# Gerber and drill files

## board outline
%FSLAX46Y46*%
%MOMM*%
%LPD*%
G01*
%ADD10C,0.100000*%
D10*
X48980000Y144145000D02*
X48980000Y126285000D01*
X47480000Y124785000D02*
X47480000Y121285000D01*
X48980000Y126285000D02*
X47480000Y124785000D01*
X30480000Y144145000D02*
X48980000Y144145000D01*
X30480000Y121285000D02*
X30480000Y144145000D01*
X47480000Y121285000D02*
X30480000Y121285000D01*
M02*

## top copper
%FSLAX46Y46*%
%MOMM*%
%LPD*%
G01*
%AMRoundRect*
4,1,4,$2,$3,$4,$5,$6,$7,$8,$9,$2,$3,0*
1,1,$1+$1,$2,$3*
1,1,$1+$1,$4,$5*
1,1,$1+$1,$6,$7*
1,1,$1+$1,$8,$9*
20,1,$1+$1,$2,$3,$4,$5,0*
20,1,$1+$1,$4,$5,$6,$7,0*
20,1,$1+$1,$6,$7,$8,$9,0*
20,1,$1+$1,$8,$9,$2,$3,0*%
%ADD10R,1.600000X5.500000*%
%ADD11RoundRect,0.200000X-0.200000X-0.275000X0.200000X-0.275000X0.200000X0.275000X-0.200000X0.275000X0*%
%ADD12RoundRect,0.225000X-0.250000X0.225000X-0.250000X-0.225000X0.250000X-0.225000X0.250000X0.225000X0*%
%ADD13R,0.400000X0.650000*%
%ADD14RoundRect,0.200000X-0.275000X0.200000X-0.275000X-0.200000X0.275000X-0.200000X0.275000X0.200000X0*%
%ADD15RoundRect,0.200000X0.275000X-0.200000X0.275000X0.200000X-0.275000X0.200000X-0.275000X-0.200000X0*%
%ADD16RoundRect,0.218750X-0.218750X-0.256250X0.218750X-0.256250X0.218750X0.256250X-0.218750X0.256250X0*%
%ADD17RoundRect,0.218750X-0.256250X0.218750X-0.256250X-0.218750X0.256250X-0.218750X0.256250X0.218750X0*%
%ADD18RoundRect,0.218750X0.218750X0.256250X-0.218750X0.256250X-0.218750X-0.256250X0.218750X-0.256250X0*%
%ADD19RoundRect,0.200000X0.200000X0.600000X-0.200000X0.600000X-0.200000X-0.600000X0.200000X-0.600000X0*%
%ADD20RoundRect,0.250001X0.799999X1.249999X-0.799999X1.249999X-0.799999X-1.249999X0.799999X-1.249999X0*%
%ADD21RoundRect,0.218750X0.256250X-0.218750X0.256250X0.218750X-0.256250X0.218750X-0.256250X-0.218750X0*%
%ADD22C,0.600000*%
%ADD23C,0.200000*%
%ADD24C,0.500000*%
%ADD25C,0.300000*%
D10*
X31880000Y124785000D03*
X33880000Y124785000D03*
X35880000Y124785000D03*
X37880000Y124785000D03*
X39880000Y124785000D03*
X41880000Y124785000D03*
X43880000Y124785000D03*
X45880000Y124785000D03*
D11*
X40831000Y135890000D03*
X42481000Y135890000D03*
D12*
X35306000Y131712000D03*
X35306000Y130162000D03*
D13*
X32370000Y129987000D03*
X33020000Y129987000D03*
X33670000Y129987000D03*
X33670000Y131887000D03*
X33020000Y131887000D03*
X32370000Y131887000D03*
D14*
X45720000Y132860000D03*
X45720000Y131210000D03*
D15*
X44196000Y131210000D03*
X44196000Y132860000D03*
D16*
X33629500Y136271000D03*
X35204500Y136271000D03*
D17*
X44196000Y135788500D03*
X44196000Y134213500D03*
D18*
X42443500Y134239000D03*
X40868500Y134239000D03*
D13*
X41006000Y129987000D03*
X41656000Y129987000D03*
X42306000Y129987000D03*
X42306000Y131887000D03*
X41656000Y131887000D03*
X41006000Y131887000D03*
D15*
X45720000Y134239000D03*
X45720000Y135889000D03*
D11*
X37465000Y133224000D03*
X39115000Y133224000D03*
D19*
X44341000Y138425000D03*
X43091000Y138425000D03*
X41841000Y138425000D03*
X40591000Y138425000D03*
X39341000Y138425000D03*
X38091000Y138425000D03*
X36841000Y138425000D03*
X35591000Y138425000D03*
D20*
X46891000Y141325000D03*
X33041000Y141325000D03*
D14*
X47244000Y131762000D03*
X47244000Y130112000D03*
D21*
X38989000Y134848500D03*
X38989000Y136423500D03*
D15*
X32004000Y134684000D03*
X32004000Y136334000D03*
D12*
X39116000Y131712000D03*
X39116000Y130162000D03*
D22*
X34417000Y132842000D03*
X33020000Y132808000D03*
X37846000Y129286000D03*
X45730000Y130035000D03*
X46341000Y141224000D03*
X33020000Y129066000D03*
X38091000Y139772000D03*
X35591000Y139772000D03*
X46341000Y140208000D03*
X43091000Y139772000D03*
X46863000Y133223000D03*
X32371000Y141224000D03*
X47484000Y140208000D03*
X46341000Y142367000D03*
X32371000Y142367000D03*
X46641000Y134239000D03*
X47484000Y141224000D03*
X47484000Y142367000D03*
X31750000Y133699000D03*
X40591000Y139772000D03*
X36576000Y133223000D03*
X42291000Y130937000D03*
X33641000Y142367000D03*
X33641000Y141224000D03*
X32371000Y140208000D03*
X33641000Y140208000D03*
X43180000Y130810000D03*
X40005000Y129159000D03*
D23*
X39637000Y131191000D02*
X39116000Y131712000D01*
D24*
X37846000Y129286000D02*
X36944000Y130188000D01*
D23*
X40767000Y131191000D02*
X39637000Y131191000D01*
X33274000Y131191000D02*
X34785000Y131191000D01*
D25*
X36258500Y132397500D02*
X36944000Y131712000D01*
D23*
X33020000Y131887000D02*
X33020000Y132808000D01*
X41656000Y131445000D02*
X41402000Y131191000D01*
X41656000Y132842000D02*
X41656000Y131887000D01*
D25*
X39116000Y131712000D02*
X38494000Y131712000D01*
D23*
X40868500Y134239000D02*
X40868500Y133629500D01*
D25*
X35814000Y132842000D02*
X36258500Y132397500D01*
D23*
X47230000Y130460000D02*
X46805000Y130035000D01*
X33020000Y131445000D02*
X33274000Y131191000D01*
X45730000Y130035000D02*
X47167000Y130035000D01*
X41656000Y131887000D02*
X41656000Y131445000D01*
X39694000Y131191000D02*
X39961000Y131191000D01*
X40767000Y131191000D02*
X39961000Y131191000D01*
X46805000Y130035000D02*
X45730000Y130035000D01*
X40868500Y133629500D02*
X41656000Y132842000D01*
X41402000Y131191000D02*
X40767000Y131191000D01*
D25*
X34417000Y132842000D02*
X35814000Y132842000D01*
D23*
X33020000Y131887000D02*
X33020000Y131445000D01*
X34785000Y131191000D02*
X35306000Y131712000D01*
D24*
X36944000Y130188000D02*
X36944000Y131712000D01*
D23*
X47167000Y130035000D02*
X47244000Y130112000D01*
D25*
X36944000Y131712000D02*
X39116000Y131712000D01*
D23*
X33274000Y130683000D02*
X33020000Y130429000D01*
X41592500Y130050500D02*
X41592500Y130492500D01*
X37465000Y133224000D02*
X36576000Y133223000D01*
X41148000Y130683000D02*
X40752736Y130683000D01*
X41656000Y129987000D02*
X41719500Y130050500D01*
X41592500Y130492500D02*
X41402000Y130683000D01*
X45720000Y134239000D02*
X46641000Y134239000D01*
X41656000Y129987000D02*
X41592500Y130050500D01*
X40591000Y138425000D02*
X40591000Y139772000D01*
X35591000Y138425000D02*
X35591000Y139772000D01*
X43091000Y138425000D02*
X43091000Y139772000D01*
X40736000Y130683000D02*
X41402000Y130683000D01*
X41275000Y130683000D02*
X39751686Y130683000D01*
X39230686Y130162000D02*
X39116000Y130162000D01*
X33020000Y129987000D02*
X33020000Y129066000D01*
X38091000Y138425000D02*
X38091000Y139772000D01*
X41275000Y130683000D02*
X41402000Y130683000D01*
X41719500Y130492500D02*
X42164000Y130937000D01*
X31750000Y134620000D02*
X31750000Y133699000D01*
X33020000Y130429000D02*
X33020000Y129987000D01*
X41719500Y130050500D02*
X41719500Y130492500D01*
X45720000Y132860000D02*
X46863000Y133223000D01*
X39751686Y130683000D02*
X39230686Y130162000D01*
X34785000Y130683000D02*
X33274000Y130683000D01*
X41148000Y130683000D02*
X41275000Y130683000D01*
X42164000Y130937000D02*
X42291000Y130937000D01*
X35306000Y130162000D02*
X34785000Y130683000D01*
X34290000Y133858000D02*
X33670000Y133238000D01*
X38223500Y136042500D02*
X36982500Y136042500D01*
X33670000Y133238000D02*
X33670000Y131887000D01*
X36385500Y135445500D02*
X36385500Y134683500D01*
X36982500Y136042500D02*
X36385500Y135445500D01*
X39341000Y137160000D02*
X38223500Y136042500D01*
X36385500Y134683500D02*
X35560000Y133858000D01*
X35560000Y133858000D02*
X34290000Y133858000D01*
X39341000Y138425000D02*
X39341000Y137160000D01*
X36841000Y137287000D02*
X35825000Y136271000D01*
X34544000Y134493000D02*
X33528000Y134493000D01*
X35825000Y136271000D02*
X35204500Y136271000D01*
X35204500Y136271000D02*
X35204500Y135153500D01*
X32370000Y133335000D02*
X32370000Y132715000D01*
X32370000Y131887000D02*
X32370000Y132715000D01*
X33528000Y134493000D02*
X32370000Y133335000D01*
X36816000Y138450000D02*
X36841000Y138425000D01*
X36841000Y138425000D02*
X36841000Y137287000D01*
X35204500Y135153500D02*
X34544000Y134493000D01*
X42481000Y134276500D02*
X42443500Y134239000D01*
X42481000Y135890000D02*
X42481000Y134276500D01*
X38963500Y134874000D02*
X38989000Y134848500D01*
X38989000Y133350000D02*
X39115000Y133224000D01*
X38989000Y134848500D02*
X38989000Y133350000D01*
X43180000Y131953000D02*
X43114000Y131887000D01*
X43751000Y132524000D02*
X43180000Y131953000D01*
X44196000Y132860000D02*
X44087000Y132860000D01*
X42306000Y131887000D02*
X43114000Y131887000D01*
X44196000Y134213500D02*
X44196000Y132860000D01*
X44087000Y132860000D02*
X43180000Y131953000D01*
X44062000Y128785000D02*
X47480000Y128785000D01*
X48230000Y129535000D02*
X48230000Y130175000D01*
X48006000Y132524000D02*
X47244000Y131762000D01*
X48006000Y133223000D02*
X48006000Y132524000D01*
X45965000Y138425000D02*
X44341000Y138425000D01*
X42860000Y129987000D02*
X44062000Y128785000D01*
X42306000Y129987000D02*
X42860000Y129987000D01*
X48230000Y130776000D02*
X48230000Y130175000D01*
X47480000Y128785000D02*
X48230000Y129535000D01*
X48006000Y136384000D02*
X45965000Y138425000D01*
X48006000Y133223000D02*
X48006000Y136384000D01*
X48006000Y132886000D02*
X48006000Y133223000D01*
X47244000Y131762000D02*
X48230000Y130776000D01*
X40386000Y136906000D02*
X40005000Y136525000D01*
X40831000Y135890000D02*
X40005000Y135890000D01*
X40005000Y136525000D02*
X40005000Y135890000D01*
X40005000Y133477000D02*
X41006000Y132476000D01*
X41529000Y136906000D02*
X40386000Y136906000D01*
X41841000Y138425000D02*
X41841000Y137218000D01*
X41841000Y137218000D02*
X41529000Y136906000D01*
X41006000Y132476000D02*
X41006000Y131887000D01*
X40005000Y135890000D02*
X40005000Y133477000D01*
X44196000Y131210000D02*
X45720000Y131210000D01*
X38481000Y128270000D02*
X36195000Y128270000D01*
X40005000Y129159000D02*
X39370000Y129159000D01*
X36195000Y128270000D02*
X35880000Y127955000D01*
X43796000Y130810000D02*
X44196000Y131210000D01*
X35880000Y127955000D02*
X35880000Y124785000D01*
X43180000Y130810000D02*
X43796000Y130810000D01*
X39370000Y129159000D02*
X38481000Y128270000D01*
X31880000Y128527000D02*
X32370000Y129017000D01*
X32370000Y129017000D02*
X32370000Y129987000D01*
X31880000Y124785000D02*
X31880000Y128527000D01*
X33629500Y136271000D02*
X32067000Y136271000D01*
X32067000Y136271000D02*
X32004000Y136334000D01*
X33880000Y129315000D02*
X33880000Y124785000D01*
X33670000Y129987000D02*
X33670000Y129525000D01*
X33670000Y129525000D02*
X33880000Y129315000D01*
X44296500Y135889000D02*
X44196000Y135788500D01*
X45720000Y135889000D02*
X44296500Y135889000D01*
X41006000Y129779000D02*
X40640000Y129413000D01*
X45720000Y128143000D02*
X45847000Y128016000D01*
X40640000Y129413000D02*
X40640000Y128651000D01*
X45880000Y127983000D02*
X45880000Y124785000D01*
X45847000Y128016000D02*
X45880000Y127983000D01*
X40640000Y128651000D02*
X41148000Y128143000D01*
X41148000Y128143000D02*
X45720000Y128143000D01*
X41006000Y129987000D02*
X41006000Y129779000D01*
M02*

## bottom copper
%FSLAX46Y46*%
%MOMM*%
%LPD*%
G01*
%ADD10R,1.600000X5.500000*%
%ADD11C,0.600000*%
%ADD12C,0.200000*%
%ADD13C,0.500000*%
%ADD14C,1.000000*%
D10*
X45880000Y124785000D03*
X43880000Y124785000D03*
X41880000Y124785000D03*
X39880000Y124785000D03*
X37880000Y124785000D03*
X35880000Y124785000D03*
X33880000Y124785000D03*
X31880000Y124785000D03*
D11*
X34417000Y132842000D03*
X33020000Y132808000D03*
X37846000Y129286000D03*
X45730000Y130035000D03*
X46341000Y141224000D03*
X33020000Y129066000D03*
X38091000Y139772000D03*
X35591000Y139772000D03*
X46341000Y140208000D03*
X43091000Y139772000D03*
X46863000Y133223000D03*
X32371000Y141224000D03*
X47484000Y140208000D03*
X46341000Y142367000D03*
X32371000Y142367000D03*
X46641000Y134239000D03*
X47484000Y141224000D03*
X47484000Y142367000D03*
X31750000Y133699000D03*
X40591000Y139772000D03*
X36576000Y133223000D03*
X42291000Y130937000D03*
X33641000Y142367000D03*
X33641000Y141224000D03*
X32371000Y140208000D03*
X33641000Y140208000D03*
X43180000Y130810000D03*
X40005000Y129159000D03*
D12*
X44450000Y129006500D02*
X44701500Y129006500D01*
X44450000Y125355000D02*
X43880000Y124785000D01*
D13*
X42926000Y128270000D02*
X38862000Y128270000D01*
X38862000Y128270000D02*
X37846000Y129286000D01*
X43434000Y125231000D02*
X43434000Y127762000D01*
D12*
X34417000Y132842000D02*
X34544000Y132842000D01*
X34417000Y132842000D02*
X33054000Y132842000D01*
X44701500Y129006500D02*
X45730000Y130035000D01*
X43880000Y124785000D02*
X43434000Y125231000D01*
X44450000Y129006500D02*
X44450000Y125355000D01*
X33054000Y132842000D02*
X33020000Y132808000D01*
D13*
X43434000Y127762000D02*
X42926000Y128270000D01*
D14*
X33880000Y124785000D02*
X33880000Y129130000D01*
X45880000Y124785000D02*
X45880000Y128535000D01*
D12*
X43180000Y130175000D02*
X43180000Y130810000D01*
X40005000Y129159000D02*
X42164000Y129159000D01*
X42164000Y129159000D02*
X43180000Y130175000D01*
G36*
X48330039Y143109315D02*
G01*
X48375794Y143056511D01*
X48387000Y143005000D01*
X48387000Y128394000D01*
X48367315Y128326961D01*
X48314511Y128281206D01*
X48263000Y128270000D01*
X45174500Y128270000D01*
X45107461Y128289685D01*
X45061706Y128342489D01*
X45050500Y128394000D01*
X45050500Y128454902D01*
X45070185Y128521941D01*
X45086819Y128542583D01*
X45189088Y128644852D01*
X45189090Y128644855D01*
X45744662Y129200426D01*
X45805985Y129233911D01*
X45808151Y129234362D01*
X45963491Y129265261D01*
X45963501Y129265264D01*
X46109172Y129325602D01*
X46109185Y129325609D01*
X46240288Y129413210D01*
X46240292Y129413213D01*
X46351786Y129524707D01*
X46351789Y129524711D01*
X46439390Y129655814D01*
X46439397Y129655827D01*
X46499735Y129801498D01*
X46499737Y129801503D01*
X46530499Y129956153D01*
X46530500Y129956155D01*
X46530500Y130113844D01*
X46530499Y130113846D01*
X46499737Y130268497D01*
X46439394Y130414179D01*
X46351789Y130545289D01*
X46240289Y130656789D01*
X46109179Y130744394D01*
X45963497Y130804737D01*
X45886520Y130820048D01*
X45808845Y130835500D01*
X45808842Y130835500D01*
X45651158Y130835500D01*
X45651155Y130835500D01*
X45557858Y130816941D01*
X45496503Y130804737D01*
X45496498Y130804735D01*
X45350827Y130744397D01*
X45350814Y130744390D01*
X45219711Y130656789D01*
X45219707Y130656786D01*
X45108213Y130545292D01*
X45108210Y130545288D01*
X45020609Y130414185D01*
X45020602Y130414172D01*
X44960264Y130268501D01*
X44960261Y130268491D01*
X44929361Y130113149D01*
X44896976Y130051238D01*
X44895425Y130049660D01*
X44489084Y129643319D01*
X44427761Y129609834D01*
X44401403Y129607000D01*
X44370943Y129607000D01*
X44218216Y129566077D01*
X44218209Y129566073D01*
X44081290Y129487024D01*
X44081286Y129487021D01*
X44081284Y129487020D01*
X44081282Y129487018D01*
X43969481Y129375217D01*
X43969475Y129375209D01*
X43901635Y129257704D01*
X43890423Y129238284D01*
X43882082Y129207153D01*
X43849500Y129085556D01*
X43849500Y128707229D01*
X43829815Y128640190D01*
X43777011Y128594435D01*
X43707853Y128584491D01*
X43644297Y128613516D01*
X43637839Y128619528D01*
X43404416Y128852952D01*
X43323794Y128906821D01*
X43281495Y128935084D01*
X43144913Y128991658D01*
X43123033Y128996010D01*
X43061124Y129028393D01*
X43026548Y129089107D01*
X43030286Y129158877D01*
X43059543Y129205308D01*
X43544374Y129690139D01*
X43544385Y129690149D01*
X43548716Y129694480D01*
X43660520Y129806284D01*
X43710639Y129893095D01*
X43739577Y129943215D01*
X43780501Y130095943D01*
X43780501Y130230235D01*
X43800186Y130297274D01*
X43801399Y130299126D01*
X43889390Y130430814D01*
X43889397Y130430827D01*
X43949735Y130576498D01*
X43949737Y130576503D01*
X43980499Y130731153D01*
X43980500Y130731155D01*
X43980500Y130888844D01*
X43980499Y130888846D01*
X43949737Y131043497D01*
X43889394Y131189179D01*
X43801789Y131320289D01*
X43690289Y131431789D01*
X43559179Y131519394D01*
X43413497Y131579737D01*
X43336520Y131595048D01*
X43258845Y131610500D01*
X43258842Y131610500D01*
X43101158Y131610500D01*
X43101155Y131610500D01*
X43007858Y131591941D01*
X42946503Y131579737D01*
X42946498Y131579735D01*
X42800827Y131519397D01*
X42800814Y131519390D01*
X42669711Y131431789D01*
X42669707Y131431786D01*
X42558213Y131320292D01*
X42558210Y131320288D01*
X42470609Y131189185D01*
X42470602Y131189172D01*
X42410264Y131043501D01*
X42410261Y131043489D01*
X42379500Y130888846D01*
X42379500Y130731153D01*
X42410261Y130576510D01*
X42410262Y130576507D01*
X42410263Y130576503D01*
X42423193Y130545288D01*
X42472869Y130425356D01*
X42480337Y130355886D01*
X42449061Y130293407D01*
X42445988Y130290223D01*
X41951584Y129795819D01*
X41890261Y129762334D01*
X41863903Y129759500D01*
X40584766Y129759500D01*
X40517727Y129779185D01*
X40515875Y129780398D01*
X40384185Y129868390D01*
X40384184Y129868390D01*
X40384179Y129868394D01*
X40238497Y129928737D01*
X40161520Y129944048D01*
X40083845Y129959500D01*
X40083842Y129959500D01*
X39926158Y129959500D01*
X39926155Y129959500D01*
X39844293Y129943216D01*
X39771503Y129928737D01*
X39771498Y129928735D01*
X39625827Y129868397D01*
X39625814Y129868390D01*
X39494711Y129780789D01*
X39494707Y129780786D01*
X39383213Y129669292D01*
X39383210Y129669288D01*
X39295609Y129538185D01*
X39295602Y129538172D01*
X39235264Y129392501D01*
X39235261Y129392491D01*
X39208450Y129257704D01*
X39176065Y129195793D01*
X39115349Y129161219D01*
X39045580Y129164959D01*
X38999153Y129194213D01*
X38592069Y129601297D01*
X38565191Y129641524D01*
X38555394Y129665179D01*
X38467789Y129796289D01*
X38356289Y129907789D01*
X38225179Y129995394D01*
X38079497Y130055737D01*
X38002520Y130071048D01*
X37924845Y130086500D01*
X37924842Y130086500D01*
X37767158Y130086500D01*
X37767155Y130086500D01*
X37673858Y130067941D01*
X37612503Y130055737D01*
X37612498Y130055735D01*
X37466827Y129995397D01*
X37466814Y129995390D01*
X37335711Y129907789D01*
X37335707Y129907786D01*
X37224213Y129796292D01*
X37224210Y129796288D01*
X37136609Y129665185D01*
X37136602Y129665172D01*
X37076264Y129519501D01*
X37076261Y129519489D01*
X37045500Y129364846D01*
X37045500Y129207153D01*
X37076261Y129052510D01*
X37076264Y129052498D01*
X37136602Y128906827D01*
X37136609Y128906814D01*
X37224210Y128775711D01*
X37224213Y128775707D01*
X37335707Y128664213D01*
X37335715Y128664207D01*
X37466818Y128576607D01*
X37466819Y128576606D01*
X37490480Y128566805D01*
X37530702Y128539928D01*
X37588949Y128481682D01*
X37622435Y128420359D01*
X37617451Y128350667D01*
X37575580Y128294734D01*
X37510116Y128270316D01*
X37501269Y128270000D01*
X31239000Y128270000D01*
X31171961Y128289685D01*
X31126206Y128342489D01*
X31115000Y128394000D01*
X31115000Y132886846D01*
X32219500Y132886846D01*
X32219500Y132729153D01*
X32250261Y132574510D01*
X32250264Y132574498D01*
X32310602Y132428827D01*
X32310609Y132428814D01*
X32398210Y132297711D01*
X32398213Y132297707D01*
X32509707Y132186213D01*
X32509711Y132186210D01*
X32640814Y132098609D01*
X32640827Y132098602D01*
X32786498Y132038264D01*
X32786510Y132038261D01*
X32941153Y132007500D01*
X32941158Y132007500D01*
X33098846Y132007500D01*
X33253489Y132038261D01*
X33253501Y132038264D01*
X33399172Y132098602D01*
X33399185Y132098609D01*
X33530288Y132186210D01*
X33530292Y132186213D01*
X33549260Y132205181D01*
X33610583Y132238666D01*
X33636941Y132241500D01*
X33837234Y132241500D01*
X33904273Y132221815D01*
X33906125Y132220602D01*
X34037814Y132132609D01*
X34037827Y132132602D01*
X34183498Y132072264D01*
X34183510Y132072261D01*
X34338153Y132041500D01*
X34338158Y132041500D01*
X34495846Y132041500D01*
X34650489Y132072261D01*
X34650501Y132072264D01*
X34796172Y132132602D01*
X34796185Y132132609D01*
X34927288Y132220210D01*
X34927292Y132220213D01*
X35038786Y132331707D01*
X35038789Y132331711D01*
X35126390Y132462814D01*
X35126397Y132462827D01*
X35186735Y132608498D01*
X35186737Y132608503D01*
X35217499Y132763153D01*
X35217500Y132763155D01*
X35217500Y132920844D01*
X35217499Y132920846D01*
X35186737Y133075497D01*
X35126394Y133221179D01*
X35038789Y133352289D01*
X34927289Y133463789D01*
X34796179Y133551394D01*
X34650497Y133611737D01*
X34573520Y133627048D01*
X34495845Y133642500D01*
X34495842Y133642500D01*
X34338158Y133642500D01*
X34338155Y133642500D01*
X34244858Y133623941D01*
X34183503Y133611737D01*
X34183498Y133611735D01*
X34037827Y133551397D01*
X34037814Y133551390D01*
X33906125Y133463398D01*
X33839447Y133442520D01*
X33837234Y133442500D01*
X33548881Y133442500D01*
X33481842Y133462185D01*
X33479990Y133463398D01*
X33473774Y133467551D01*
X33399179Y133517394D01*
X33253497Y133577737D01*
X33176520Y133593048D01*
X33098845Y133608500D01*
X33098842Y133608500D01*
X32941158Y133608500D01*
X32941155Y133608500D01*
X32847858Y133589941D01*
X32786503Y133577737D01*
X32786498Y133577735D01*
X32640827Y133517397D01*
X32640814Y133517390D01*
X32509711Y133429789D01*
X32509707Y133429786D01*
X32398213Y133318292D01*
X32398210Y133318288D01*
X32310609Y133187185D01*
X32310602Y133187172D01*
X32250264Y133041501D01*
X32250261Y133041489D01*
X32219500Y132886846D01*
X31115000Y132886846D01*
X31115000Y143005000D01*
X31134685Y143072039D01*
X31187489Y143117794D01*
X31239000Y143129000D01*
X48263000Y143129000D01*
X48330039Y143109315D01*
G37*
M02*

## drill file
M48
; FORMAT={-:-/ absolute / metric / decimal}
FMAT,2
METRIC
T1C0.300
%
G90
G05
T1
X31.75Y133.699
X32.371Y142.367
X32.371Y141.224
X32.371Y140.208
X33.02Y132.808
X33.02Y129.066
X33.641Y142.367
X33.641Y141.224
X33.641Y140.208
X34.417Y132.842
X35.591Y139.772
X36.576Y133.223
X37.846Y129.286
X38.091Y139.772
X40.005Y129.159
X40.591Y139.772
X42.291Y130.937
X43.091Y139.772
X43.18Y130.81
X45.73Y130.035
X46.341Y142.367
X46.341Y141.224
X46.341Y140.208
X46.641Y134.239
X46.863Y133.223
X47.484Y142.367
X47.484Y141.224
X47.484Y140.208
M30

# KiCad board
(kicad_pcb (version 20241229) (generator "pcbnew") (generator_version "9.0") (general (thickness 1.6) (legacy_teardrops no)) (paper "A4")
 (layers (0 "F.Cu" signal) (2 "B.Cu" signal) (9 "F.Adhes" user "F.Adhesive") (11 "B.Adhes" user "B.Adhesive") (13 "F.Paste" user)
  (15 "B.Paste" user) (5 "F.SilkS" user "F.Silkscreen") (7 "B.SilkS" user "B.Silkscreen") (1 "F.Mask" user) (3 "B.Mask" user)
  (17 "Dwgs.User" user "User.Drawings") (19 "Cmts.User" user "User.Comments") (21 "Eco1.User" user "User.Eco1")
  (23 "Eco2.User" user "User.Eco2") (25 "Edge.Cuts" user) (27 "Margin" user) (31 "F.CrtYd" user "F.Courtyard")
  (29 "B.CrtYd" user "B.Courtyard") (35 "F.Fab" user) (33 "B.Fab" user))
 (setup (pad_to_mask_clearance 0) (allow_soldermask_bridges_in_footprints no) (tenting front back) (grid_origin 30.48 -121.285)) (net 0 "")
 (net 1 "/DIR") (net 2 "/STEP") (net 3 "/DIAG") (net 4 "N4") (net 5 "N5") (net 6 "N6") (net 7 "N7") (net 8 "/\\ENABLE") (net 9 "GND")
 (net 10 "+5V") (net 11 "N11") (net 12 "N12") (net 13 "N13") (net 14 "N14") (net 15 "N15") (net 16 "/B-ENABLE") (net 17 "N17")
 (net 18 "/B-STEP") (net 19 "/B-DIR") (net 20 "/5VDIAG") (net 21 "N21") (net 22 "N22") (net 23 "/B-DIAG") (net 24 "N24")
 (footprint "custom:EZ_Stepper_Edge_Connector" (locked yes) (layer "F.Cu") (at 30.48 -121.285)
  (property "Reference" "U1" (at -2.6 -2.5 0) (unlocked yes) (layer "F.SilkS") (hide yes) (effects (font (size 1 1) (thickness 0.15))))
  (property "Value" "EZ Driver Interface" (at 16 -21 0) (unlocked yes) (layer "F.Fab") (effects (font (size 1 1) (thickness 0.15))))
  (pad "1" smd rect (at 1.4 -3.5) (size 1.6 5.5) (layers "F.Cu" "F.Mask" "F.Paste") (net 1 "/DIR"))
  (pad "2" smd rect (at 3.4 -3.5) (size 1.6 5.5) (layers "F.Cu" "F.Mask" "F.Paste") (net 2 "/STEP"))
  (pad "3" smd rect (at 5.4 -3.5) (size 1.6 5.5) (layers "F.Cu" "F.Mask" "F.Paste") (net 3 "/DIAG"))
  (pad "4" smd rect (at 7.4 -3.5) (size 1.6 5.5) (layers "F.Cu" "F.Mask" "F.Paste") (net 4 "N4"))
  (pad "5" smd rect (at 9.4 -3.5) (size 1.6 5.5) (layers "F.Cu" "F.Mask" "F.Paste") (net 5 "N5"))
  (pad "6" smd rect (at 11.4 -3.5) (size 1.6 5.5) (layers "F.Cu" "F.Mask" "F.Paste") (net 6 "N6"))
  (pad "7" smd rect (at 13.4 -3.5) (size 1.6 5.5) (layers "F.Cu" "F.Mask" "F.Paste") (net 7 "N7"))
  (pad "8" smd rect (at 15.4 -3.5) (size 1.6 5.5) (layers "F.Cu" "F.Mask" "F.Paste") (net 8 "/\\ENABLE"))
  (pad "9" smd rect (at 15.4 -3.5) (size 1.6 5.5) (layers "B.Cu" "B.Mask" "B.Paste") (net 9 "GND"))
  (pad "10" smd rect (at 13.4 -3.5) (size 1.6 5.5) (layers "B.Cu" "B.Mask" "B.Paste") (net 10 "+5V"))
  (pad "11" smd rect (at 11.4 -3.5) (size 1.6 5.5) (layers "B.Cu" "B.Mask" "B.Paste") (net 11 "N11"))
  (pad "12" smd rect (at 9.4 -3.5) (size 1.6 5.5) (layers "B.Cu" "B.Mask" "B.Paste") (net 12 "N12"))
  (pad "13" smd rect (at 7.4 -3.5) (size 1.6 5.5) (layers "B.Cu" "B.Mask" "B.Paste") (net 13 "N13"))
  (pad "14" smd rect (at 5.4 -3.5) (size 1.6 5.5) (layers "B.Cu" "B.Mask" "B.Paste") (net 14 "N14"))
  (pad "15" smd rect (at 3.4 -3.5) (size 1.6 5.5) (layers "B.Cu" "B.Mask" "B.Paste") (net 9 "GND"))
  (pad "16" smd rect (at 1.4 -3.5) (size 1.6 5.5) (layers "B.Cu" "B.Mask" "B.Paste") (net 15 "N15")))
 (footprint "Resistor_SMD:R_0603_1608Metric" (layer "F.Cu") (at 41.656 -135.89)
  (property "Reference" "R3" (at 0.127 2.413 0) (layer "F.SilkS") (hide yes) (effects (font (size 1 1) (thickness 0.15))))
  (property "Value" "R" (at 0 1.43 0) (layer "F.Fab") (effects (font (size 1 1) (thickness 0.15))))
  (pad "1" smd roundrect (at -0.825 0) (size 0.8 0.95) (layers "F.Cu" "F.Mask" "F.Paste") (roundrect_rratio 0.25) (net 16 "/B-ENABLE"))
  (pad "2" smd roundrect (at 0.825 0) (size 0.8 0.95) (layers "F.Cu" "F.Mask" "F.Paste") (roundrect_rratio 0.25) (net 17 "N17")))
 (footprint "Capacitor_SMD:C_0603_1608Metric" (layer "F.Cu") (at 35.306 -130.937 -90)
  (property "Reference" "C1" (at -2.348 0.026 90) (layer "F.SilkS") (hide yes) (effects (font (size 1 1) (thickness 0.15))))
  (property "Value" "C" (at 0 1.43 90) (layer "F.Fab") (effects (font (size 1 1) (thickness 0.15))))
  (pad "1" smd roundrect (at -0.775 0 270) (size 0.9 0.95) (layers "F.Cu" "F.Mask" "F.Paste") (roundrect_rratio 0.25) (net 10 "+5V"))
  (pad "2" smd roundrect (at 0.775 0 270) (size 0.9 0.95) (layers "F.Cu" "F.Mask" "F.Paste") (roundrect_rratio 0.25) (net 9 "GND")))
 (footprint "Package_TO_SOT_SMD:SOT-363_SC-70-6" (layer "F.Cu") (at 33.02 -130.937 90)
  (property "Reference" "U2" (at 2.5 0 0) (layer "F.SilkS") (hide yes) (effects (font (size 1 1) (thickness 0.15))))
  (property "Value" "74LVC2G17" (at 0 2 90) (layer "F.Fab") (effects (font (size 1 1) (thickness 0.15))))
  (pad "1" smd rect (at -0.95 -0.65 90) (size 0.65 0.4) (layers "F.Cu" "F.Mask" "F.Paste") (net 1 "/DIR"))
  (pad "2" smd rect (at -0.95 0 90) (size 0.65 0.4) (layers "F.Cu" "F.Mask" "F.Paste") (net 9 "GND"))
  (pad "3" smd rect (at -0.95 0.65 90) (size 0.65 0.4) (layers "F.Cu" "F.Mask" "F.Paste") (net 2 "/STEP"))
  (pad "4" smd rect (at 0.95 0.65 90) (size 0.65 0.4) (layers "F.Cu" "F.Mask" "F.Paste") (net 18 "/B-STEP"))
  (pad "5" smd rect (at 0.95 0 90) (size 0.65 0.4) (layers "F.Cu" "F.Mask" "F.Paste") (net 10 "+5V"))
  (pad "6" smd rect (at 0.95 -0.65 90) (size 0.65 0.4) (layers "F.Cu" "F.Mask" "F.Paste") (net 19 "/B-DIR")))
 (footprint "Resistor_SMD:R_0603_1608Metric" (layer "F.Cu") (at 45.72 -132.035 -90)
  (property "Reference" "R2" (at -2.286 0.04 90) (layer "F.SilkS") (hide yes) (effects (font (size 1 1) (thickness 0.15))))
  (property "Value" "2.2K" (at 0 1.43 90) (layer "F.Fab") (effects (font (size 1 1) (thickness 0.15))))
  (pad "1" smd roundrect (at -0.825 0 270) (size 0.8 0.95) (layers "F.Cu" "F.Mask" "F.Paste") (roundrect_rratio 0.25) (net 9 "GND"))
  (pad "2" smd roundrect (at 0.825 0 270) (size 0.8 0.95) (layers "F.Cu" "F.Mask" "F.Paste") (roundrect_rratio 0.25) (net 3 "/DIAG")))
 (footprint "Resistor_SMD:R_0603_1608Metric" (layer "F.Cu") (at 44.196 -132.035 90)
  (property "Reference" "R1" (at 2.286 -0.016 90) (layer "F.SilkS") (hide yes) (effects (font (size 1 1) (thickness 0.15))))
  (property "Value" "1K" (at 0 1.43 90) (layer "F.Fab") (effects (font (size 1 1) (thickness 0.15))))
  (pad "1" smd roundrect (at -0.825 0 90) (size 0.8 0.95) (layers "F.Cu" "F.Mask" "F.Paste") (roundrect_rratio 0.25) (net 3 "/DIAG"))
  (pad "2" smd roundrect (at 0.825 0 90) (size 0.8 0.95) (layers "F.Cu" "F.Mask" "F.Paste") (roundrect_rratio 0.25) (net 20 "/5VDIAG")))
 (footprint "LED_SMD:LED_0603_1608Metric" (layer "F.Cu") (at 34.417 -136.271)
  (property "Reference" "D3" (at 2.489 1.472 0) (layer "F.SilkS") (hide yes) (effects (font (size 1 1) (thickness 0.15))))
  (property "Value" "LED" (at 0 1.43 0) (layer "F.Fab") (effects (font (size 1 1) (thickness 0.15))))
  (pad "1" smd roundrect (at -0.7875 0) (size 0.875 0.95) (layers "F.Cu" "F.Mask" "F.Paste") (roundrect_rratio 0.25) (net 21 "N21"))
  (pad "2" smd roundrect (at 0.7875 0) (size 0.875 0.95) (layers "F.Cu" "F.Mask" "F.Paste") (roundrect_rratio 0.25) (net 19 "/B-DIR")))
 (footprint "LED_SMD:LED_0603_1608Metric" (layer "F.Cu") (at 44.196 -135.001 -90)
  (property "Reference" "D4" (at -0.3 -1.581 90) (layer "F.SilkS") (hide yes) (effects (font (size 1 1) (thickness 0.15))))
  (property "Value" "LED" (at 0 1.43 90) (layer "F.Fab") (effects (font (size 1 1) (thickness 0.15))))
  (pad "1" smd roundrect (at -0.7875 0 270) (size 0.875 0.95) (layers "F.Cu" "F.Mask" "F.Paste") (roundrect_rratio 0.25) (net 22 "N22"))
  (pad "2" smd roundrect (at 0.7875 0 270) (size 0.875 0.95) (layers "F.Cu" "F.Mask" "F.Paste") (roundrect_rratio 0.25) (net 20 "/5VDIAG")))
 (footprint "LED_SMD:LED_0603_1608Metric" (layer "F.Cu") (at 41.656 -134.239 180)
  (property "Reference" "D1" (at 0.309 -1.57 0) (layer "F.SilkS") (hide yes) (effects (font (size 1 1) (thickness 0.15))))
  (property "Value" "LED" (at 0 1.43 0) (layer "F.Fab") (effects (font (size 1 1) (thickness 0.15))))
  (pad "1" smd roundrect (at -0.7875 0 180) (size 0.875 0.95) (layers "F.Cu" "F.Mask" "F.Paste") (roundrect_rratio 0.25) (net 17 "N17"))
  (pad "2" smd roundrect (at 0.7875 0 180) (size 0.875 0.95) (layers "F.Cu" "F.Mask" "F.Paste") (roundrect_rratio 0.25) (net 10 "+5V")))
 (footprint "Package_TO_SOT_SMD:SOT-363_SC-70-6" (layer "F.Cu") (at 41.656 -130.937 90)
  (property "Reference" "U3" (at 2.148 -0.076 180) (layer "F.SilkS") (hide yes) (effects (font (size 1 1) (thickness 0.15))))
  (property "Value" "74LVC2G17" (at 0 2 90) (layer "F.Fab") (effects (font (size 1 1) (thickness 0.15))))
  (pad "1" smd rect (at -0.95 -0.65 90) (size 0.65 0.4) (layers "F.Cu" "F.Mask" "F.Paste") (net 8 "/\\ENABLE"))
  (pad "2" smd rect (at -0.95 0 90) (size 0.65 0.4) (layers "F.Cu" "F.Mask" "F.Paste") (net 9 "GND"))
  (pad "3" smd rect (at -0.95 0.65 90) (size 0.65 0.4) (layers "F.Cu" "F.Mask" "F.Paste") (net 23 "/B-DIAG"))
  (pad "4" smd rect (at 0.95 0.65 90) (size 0.65 0.4) (layers "F.Cu" "F.Mask" "F.Paste") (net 20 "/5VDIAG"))
  (pad "5" smd rect (at 0.95 0 90) (size 0.65 0.4) (layers "F.Cu" "F.Mask" "F.Paste") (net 10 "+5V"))
  (pad "6" smd rect (at 0.95 -0.65 90) (size 0.65 0.4) (layers "F.Cu" "F.Mask" "F.Paste") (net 16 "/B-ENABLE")))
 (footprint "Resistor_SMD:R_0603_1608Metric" (layer "F.Cu") (at 45.72 -135.064 90)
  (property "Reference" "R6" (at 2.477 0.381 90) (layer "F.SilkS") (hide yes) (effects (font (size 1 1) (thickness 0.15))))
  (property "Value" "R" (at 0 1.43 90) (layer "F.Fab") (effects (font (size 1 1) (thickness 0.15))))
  (pad "1" smd roundrect (at -0.825 0 90) (size 0.8 0.95) (layers "F.Cu" "F.Mask" "F.Paste") (roundrect_rratio 0.25) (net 9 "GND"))
  (pad "2" smd roundrect (at 0.825 0 90) (size 0.8 0.95) (layers "F.Cu" "F.Mask" "F.Paste") (roundrect_rratio 0.25) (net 22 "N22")))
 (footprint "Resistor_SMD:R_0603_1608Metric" (layer "F.Cu") (at 38.29 -133.224)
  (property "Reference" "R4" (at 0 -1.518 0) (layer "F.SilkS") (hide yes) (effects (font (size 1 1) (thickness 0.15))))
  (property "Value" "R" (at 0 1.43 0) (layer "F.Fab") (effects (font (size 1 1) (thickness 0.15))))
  (pad "1" smd roundrect (at -0.825 0) (size 0.8 0.95) (layers "F.Cu" "F.Mask" "F.Paste") (roundrect_rratio 0.25) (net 9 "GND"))
  (pad "2" smd roundrect (at 0.825 0) (size 0.8 0.95) (layers "F.Cu" "F.Mask" "F.Paste") (roundrect_rratio 0.25) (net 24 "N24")))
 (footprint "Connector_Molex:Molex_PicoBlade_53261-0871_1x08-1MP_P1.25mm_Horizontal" (layer "F.Cu") (at 39.966 -140.825 180)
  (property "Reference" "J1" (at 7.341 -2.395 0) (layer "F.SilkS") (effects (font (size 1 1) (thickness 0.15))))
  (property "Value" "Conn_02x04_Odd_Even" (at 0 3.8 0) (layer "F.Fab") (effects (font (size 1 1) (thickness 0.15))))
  (pad "1" smd roundrect (at -4.375 -2.4 180) (size 0.8 1.6) (layers "F.Cu" "F.Mask" "F.Paste") (roundrect_rratio 0.25) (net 23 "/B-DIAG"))
  (pad "2" smd roundrect (at -3.125 -2.4 180) (size 0.8 1.6) (layers "F.Cu" "F.Mask" "F.Paste") (roundrect_rratio 0.25) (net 9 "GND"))
  (pad "3" smd roundrect (at -1.875 -2.4 180) (size 0.8 1.6) (layers "F.Cu" "F.Mask" "F.Paste") (roundrect_rratio 0.25) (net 16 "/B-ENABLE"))
  (pad "4" smd roundrect (at -0.625 -2.4 180) (size 0.8 1.6) (layers "F.Cu" "F.Mask" "F.Paste") (roundrect_rratio 0.25) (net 9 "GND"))
  (pad "5" smd roundrect (at 0.625 -2.4 180) (size 0.8 1.6) (layers "F.Cu" "F.Mask" "F.Paste") (roundrect_rratio 0.25) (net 18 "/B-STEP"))
  (pad "6" smd roundrect (at 1.875 -2.4 180) (size 0.8 1.6) (layers "F.Cu" "F.Mask" "F.Paste") (roundrect_rratio 0.25) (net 9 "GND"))
  (pad "7" smd roundrect (at 3.125 -2.4 180) (size 0.8 1.6) (layers "F.Cu" "F.Mask" "F.Paste") (roundrect_rratio 0.25) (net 19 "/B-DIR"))
  (pad "8" smd roundrect (at 4.375 -2.4 180) (size 0.8 1.6) (layers "F.Cu" "F.Mask" "F.Paste") (roundrect_rratio 0.25) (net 9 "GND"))
  (pad "MP" smd roundrect (at -6.925 0.5 180) (size 2.1 3) (layers "F.Cu" "F.Mask" "F.Paste") (roundrect_rratio 0.1190480952) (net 9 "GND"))
  (pad "MP" smd roundrect (at 6.925 0.5 180) (size 2.1 3) (layers "F.Cu" "F.Mask" "F.Paste") (roundrect_rratio 0.1190480952) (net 9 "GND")))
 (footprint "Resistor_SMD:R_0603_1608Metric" (layer "F.Cu") (at 47.244 -130.937 -90)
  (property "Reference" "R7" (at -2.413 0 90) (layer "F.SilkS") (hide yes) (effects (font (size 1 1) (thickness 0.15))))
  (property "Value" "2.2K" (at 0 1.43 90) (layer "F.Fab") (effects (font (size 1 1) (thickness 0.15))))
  (pad "1" smd roundrect (at -0.825 0 270) (size 0.8 0.95) (layers "F.Cu" "F.Mask" "F.Paste") (roundrect_rratio 0.25) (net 23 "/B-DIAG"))
  (pad "2" smd roundrect (at 0.825 0 270) (size 0.8 0.95) (layers "F.Cu" "F.Mask" "F.Paste") (roundrect_rratio 0.25) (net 10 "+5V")))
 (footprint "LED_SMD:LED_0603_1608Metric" (layer "F.Cu") (at 38.989 -135.636 90)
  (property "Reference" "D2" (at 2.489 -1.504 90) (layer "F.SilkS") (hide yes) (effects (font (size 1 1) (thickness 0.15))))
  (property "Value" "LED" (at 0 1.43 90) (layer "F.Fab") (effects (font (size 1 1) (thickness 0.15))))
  (pad "1" smd roundrect (at -0.7875 0 90) (size 0.875 0.95) (layers "F.Cu" "F.Mask" "F.Paste") (roundrect_rratio 0.25) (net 24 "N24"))
  (pad "2" smd roundrect (at 0.7875 0 90) (size 0.875 0.95) (layers "F.Cu" "F.Mask" "F.Paste") (roundrect_rratio 0.25) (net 18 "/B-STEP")))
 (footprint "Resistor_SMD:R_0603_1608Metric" (layer "F.Cu") (at 32.004 -135.509 90)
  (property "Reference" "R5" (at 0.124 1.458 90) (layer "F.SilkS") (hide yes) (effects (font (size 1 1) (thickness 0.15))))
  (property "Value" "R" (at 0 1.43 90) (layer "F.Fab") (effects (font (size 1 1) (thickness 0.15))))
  (pad "1" smd roundrect (at -0.825 0 90) (size 0.8 0.95) (layers "F.Cu" "F.Mask" "F.Paste") (roundrect_rratio 0.25) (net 9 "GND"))
  (pad "2" smd roundrect (at 0.825 0 90) (size 0.8 0.95) (layers "F.Cu" "F.Mask" "F.Paste") (roundrect_rratio 0.25) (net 21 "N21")))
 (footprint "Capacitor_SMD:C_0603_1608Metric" (layer "F.Cu") (at 39.116 -130.937 -90)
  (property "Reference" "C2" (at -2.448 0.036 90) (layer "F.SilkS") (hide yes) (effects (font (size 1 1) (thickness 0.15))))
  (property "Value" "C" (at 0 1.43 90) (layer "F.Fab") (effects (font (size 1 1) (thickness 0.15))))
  (pad "1" smd roundrect (at -0.775 0 270) (size 0.9 0.95) (layers "F.Cu" "F.Mask" "F.Paste") (roundrect_rratio 0.25) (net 10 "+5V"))
  (pad "2" smd roundrect (at 0.775 0 270) (size 0.9 0.95) (layers "F.Cu" "F.Mask" "F.Paste") (roundrect_rratio 0.25) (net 9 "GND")))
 (gr_line (start 48.98 -144.145) (end 48.98 -126.285) (stroke (width 0.1) (type default)) (layer "Edge.Cuts"))
 (gr_line (start 47.48 -124.785) (end 47.48 -121.285) (stroke (width 0.1) (type default)) (layer "Edge.Cuts"))
 (gr_line (start 48.98 -126.285) (end 47.48 -124.785) (stroke (width 0.1) (type default)) (layer "Edge.Cuts"))
 (gr_line (start 30.48 -144.145) (end 48.98 -144.145) (stroke (width 0.1) (type default)) (layer "Edge.Cuts"))
 (gr_line (start 30.48 -121.285) (end 30.48 -144.145) (stroke (width 0.1) (type default)) (layer "Edge.Cuts"))
 (gr_line (start 47.48 -121.285) (end 30.48 -121.285) (stroke (width 0.1) (type default)) (layer "Edge.Cuts"))
 (segment (start 39.637 -131.191) (end 39.116 -131.712) (width 0.2) (layer "F.Cu") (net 10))
 (segment (start 37.846 -129.286) (end 36.944 -130.188) (width 0.5) (layer "F.Cu") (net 10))
 (segment (start 40.767 -131.191) (end 39.637 -131.191) (width 0.2) (layer "F.Cu") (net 10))
 (segment (start 33.274 -131.191) (end 34.785 -131.191) (width 0.2) (layer "F.Cu") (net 10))
 (segment (start 36.2585 -132.3975) (end 36.944 -131.712) (width 0.3) (layer "F.Cu") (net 10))
 (segment (start 33.02 -131.887) (end 33.02 -132.808) (width 0.2) (layer "F.Cu") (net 10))
 (segment (start 41.656 -131.445) (end 41.402 -131.191) (width 0.2) (layer "F.Cu") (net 10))
 (segment (start 41.656 -132.842) (end 41.656 -131.887) (width 0.2) (layer "F.Cu") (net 10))
 (segment (start 39.116 -131.712) (end 38.494 -131.712) (width 0.3) (layer "F.Cu") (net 10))
 (segment (start 40.8685 -134.239) (end 40.8685 -133.6295) (width 0.2) (layer "F.Cu") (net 10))
 (segment (start 35.814 -132.842) (end 36.2585 -132.3975) (width 0.3) (layer "F.Cu") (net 10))
 (segment (start 47.23 -130.46) (end 46.805 -130.035) (width 0.2) (layer "F.Cu") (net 10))
 (segment (start 33.02 -131.445) (end 33.274 -131.191) (width 0.2) (layer "F.Cu") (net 10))
 (segment (start 45.73 -130.035) (end 47.167 -130.035) (width 0.2) (layer "F.Cu") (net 10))
 (segment (start 41.656 -131.887) (end 41.656 -131.445) (width 0.2) (layer "F.Cu") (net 10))
 (segment (start 39.694 -131.191) (end 39.961 -131.191) (width 0.2) (layer "F.Cu") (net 10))
 (segment (start 40.767 -131.191) (end 39.961 -131.191) (width 0.2) (layer "F.Cu") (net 10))
 (segment (start 46.805 -130.035) (end 45.73 -130.035) (width 0.2) (layer "F.Cu") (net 10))
 (segment (start 40.8685 -133.6295) (end 41.656 -132.842) (width 0.2) (layer "F.Cu") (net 10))
 (segment (start 41.402 -131.191) (end 40.767 -131.191) (width 0.2) (layer "F.Cu") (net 10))
 (segment (start 34.417 -132.842) (end 35.814 -132.842) (width 0.3) (layer "F.Cu") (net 10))
 (segment (start 33.02 -131.887) (end 33.02 -131.445) (width 0.2) (layer "F.Cu") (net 10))
 (segment (start 34.785 -131.191) (end 35.306 -131.712) (width 0.2) (layer "F.Cu") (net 10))
 (segment (start 36.944 -130.188) (end 36.944 -131.712) (width 0.5) (layer "F.Cu") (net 10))
 (segment (start 47.167 -130.035) (end 47.244 -130.112) (width 0.2) (layer "F.Cu") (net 10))
 (segment (start 36.944 -131.712) (end 39.116 -131.712) (width 0.3) (layer "F.Cu") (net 10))
 (via (at 34.417 -132.842) (size 0.6) (drill 0.3) (layers "F.Cu" "B.Cu") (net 10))
 (via (at 33.02 -132.808) (size 0.6) (drill 0.3) (layers "F.Cu" "B.Cu") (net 10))
 (via (at 37.846 -129.286) (size 0.6) (drill 0.3) (layers "F.Cu" "B.Cu") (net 10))
 (via (at 45.73 -130.035) (size 0.6) (drill 0.3) (layers "F.Cu" "B.Cu") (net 10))
 (segment (start 44.45 -129.0065) (end 44.7015 -129.0065) (width 0.2) (layer "B.Cu") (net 10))
 (segment (start 44.45 -125.355) (end 43.88 -124.785) (width 0.2) (layer "B.Cu") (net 10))
 (segment (start 42.926 -128.27) (end 38.862 -128.27) (width 0.5) (layer "B.Cu") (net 10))
 (segment (start 38.862 -128.27) (end 37.846 -129.286) (width 0.5) (layer "B.Cu") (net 10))
 (segment (start 43.434 -125.231) (end 43.434 -127.762) (width 0.5) (layer "B.Cu") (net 10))
 (segment (start 34.417 -132.842) (end 34.544 -132.842) (width 0.2) (layer "B.Cu") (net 10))
 (segment (start 34.417 -132.842) (end 33.054 -132.842) (width 0.2) (layer "B.Cu") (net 10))
 (segment (start 44.7015 -129.0065) (end 45.73 -130.035) (width 0.2) (layer "B.Cu") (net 10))
 (segment (start 43.88 -124.785) (end 43.434 -125.231) (width 0.2) (layer "B.Cu") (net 10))
 (segment (start 44.45 -129.0065) (end 44.45 -125.355) (width 0.2) (layer "B.Cu") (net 10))
 (segment (start 33.054 -132.842) (end 33.02 -132.808) (width 0.2) (layer "B.Cu") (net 10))
 (segment (start 43.434 -127.762) (end 42.926 -128.27) (width 0.5) (layer "B.Cu") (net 10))
 (segment (start 33.274 -130.683) (end 33.02 -130.429) (width 0.2) (layer "F.Cu") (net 9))
 (segment (start 41.5925 -130.0505) (end 41.5925 -130.4925) (width 0.2) (layer "F.Cu") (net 9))
 (segment (start 37.465 -133.224) (end 36.576 -133.223) (width 0.2) (layer "F.Cu") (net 9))
 (segment (start 41.148 -130.683) (end 40.752736 -130.683) (width 0.2) (layer "F.Cu") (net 9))
 (segment (start 41.656 -129.987) (end 41.7195 -130.0505) (width 0.2) (layer "F.Cu") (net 9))
 (segment (start 41.5925 -130.4925) (end 41.402 -130.683) (width 0.2) (layer "F.Cu") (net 9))
 (segment (start 45.72 -134.239) (end 46.641 -134.239) (width 0.2) (layer "F.Cu") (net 9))
 (segment (start 41.656 -129.987) (end 41.5925 -130.0505) (width 0.2) (layer "F.Cu") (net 9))
 (segment (start 40.591 -138.425) (end 40.591 -139.772) (width 0.2) (layer "F.Cu") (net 9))
 (segment (start 35.591 -138.425) (end 35.591 -139.772) (width 0.2) (layer "F.Cu") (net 9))
 (segment (start 43.091 -138.425) (end 43.091 -139.772) (width 0.2) (layer "F.Cu") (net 9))
 (segment (start 40.736 -130.683) (end 41.402 -130.683) (width 0.2) (layer "F.Cu") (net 9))
 (segment (start 41.275 -130.683) (end 39.751686 -130.683) (width 0.2) (layer "F.Cu") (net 9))
 (segment (start 39.230686 -130.162) (end 39.116 -130.162) (width 0.2) (layer "F.Cu") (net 9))
 (segment (start 33.02 -129.987) (end 33.02 -129.066) (width 0.2) (layer "F.Cu") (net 9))
 (segment (start 38.091 -138.425) (end 38.091 -139.772) (width 0.2) (layer "F.Cu") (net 9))
 (segment (start 41.275 -130.683) (end 41.402 -130.683) (width 0.2) (layer "F.Cu") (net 9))
 (segment (start 41.7195 -130.4925) (end 42.164 -130.937) (width 0.2) (layer "F.Cu") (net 9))
 (segment (start 31.75 -134.62) (end 31.75 -133.699) (width 0.2) (layer "F.Cu") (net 9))
 (segment (start 33.02 -130.429) (end 33.02 -129.987) (width 0.2) (layer "F.Cu") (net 9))
 (segment (start 41.7195 -130.0505) (end 41.7195 -130.4925) (width 0.2) (layer "F.Cu") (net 9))
 (segment (start 45.72 -132.86) (end 46.863 -133.223) (width 0.2) (layer "F.Cu") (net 9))
 (segment (start 39.751686 -130.683) (end 39.230686 -130.162) (width 0.2) (layer "F.Cu") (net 9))
 (segment (start 34.785 -130.683) (end 33.274 -130.683) (width 0.2) (layer "F.Cu") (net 9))
 (segment (start 41.148 -130.683) (end 41.275 -130.683) (width 0.2) (layer "F.Cu") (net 9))
 (segment (start 42.164 -130.937) (end 42.291 -130.937) (width 0.2) (layer "F.Cu") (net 9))
 (segment (start 35.306 -130.162) (end 34.785 -130.683) (width 0.2) (layer "F.Cu") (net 9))
 (via (at 46.341 -141.224) (size 0.6) (drill 0.3) (layers "F.Cu" "B.Cu") (free yes) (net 9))
 (via (at 33.02 -129.066) (size 0.6) (drill 0.3) (layers "F.Cu" "B.Cu") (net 9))
 (via (at 38.091 -139.772) (size 0.6) (drill 0.3) (layers "F.Cu" "B.Cu") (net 9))
 (via (at 35.591 -139.772) (size 0.6) (drill 0.3) (layers "F.Cu" "B.Cu") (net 9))
 (via (at 46.341 -140.208) (size 0.6) (drill 0.3) (layers "F.Cu" "B.Cu") (free yes) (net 9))
 (via (at 43.091 -139.772) (size 0.6) (drill 0.3) (layers "F.Cu" "B.Cu") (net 9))
 (via (at 46.863 -133.223) (size 0.6) (drill 0.3) (layers "F.Cu" "B.Cu") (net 9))
 (via (at 32.371 -141.224) (size 0.6) (drill 0.3) (layers "F.Cu" "B.Cu") (free yes) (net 9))
 (via (at 47.484 -140.208) (size 0.6) (drill 0.3) (layers "F.Cu" "B.Cu") (free yes) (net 9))
 (via (at 46.341 -142.367) (size 0.6) (drill 0.3) (layers "F.Cu" "B.Cu") (free yes) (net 9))
 (via (at 32.371 -142.367) (size 0.6) (drill 0.3) (layers "F.Cu" "B.Cu") (free yes) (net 9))
 (via (at 46.641 -134.239) (size 0.6) (drill 0.3) (layers "F.Cu" "B.Cu") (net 9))
 (via (at 47.484 -141.224) (size 0.6) (drill 0.3) (layers "F.Cu" "B.Cu") (free yes) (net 9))
 (via (at 47.484 -142.367) (size 0.6) (drill 0.3) (layers "F.Cu" "B.Cu") (free yes) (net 9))
 (via (at 31.75 -133.699) (size 0.6) (drill 0.3) (layers "F.Cu" "B.Cu") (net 9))
 (via (at 40.591 -139.772) (size 0.6) (drill 0.3) (layers "F.Cu" "B.Cu") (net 9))
 (via (at 36.576 -133.223) (size 0.6) (drill 0.3) (layers "F.Cu" "B.Cu") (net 9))
 (via (at 42.291 -130.937) (size 0.6) (drill 0.3) (layers "F.Cu" "B.Cu") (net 9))
 (via (at 33.641 -142.367) (size 0.6) (drill 0.3) (layers "F.Cu" "B.Cu") (free yes) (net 9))
 (via (at 33.641 -141.224) (size 0.6) (drill 0.3) (layers "F.Cu" "B.Cu") (free yes) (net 9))
 (via (at 32.371 -140.208) (size 0.6) (drill 0.3) (layers "F.Cu" "B.Cu") (free yes) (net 9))
 (via (at 33.641 -140.208) (size 0.6) (drill 0.3) (layers "F.Cu" "B.Cu") (free yes) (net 9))
 (segment (start 33.88 -124.785) (end 33.88 -129.13) (width 1) (layer "B.Cu") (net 9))
 (segment (start 45.88 -124.785) (end 45.88 -128.535) (width 1) (layer "B.Cu") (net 9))
 (segment (start 34.29 -133.858) (end 33.67 -133.238) (width 0.2) (layer "F.Cu") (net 18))
 (segment (start 38.2235 -136.0425) (end 36.9825 -136.0425) (width 0.2) (layer "F.Cu") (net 18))
 (segment (start 33.67 -133.238) (end 33.67 -131.887) (width 0.2) (layer "F.Cu") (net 18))
 (segment (start 36.3855 -135.4455) (end 36.3855 -134.6835) (width 0.2) (layer "F.Cu") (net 18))
 (segment (start 36.9825 -136.0425) (end 36.3855 -135.4455) (width 0.2) (layer "F.Cu") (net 18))
 (segment (start 39.341 -137.16) (end 38.2235 -136.0425) (width 0.2) (layer "F.Cu") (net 18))
 (segment (start 36.3855 -134.6835) (end 35.56 -133.858) (width 0.2) (layer "F.Cu") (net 18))
 (segment (start 35.56 -133.858) (end 34.29 -133.858) (width 0.2) (layer "F.Cu") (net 18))
 (segment (start 39.341 -138.425) (end 39.341 -137.16) (width 0.2) (layer "F.Cu") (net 18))
 (segment (start 36.841 -137.287) (end 35.825 -136.271) (width 0.2) (layer "F.Cu") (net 19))
 (segment (start 34.544 -134.493) (end 33.528 -134.493) (width 0.2) (layer "F.Cu") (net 19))
 (segment (start 35.825 -136.271) (end 35.2045 -136.271) (width 0.2) (layer "F.Cu") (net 19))
 (segment (start 35.2045 -136.271) (end 35.2045 -135.1535) (width 0.2) (layer "F.Cu") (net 19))
 (segment (start 32.37 -133.335) (end 32.37 -132.715) (width 0.2) (layer "F.Cu") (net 19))
 (segment (start 32.37 -131.887) (end 32.37 -132.715) (width 0.2) (layer "F.Cu") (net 19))
 (segment (start 33.528 -134.493) (end 32.37 -133.335) (width 0.2) (layer "F.Cu") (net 19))
 (segment (start 36.816 -138.45) (end 36.841 -138.425) (width 0.2) (layer "F.Cu") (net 19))
 (segment (start 36.841 -138.425) (end 36.841 -137.287) (width 0.2) (layer "F.Cu") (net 19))
 (segment (start 35.2045 -135.1535) (end 34.544 -134.493) (width 0.2) (layer "F.Cu") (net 19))
 (segment (start 42.481 -134.2765) (end 42.4435 -134.239) (width 0.2) (layer "F.Cu") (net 17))
 (segment (start 42.481 -135.89) (end 42.481 -134.2765) (width 0.2) (layer "F.Cu") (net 17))
 (segment (start 38.9635 -134.874) (end 38.989 -134.8485) (width 0.2) (layer "F.Cu") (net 24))
 (segment (start 38.989 -133.35) (end 39.115 -133.224) (width 0.2) (layer "F.Cu") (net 24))
 (segment (start 38.989 -134.8485) (end 38.989 -133.35) (width 0.2) (layer "F.Cu") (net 24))
 (segment (start 43.18 -131.953) (end 43.114 -131.887) (width 0.2) (layer "F.Cu") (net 20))
 (segment (start 43.751 -132.524) (end 43.18 -131.953) (width 0.2) (layer "F.Cu") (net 20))
 (segment (start 44.196 -132.86) (end 44.087 -132.86) (width 0.2) (layer "F.Cu") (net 20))
 (segment (start 42.306 -131.887) (end 43.114 -131.887) (width 0.2) (layer "F.Cu") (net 20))
 (segment (start 44.196 -134.2135) (end 44.196 -132.86) (width 0.2) (layer "F.Cu") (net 20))
 (segment (start 44.087 -132.86) (end 43.18 -131.953) (width 0.2) (layer "F.Cu") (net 20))
 (segment (start 44.062 -128.785) (end 47.48 -128.785) (width 0.2) (layer "F.Cu") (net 23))
 (segment (start 48.23 -129.535) (end 48.23 -130.175) (width 0.2) (layer "F.Cu") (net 23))
 (segment (start 48.006 -132.524) (end 47.244 -131.762) (width 0.2) (layer "F.Cu") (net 23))
 (segment (start 48.006 -133.223) (end 48.006 -132.524) (width 0.2) (layer "F.Cu") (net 23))
 (segment (start 45.965 -138.425) (end 44.341 -138.425) (width 0.2) (layer "F.Cu") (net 23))
 (segment (start 42.86 -129.987) (end 44.062 -128.785) (width 0.2) (layer "F.Cu") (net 23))
 (segment (start 42.306 -129.987) (end 42.86 -129.987) (width 0.2) (layer "F.Cu") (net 23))
 (segment (start 48.23 -130.776) (end 48.23 -130.175) (width 0.2) (layer "F.Cu") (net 23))
 (segment (start 47.48 -128.785) (end 48.23 -129.535) (width 0.2) (layer "F.Cu") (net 23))
 (segment (start 48.006 -136.384) (end 45.965 -138.425) (width 0.2) (layer "F.Cu") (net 23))
 (segment (start 48.006 -133.223) (end 48.006 -136.384) (width 0.2) (layer "F.Cu") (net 23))
 (segment (start 48.006 -132.886) (end 48.006 -133.223) (width 0.2) (layer "F.Cu") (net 23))
 (segment (start 47.244 -131.762) (end 48.23 -130.776) (width 0.2) (layer "F.Cu") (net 23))
 (segment (start 40.386 -136.906) (end 40.005 -136.525) (width 0.2) (layer "F.Cu") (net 16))
 (segment (start 40.831 -135.89) (end 40.005 -135.89) (width 0.2) (layer "F.Cu") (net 16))
 (segment (start 40.005 -136.525) (end 40.005 -135.89) (width 0.2) (layer "F.Cu") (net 16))
 (segment (start 40.005 -133.477) (end 41.006 -132.476) (width 0.2) (layer "F.Cu") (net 16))
 (segment (start 41.529 -136.906) (end 40.386 -136.906) (width 0.2) (layer "F.Cu") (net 16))
 (segment (start 41.841 -138.425) (end 41.841 -137.218) (width 0.2) (layer "F.Cu") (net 16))
 (segment (start 41.841 -137.218) (end 41.529 -136.906) (width 0.2) (layer "F.Cu") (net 16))
 (segment (start 41.006 -132.476) (end 41.006 -131.887) (width 0.2) (layer "F.Cu") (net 16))
 (segment (start 40.005 -135.89) (end 40.005 -133.477) (width 0.2) (layer "F.Cu") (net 16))
 (segment (start 44.196 -131.21) (end 45.72 -131.21) (width 0.2) (layer "F.Cu") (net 3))
 (segment (start 38.481 -128.27) (end 36.195 -128.27) (width 0.2) (layer "F.Cu") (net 3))
 (segment (start 40.005 -129.159) (end 39.37 -129.159) (width 0.2) (layer "F.Cu") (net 3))
 (segment (start 36.195 -128.27) (end 35.88 -127.955) (width 0.2) (layer "F.Cu") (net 3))
 (segment (start 43.796 -130.81) (end 44.196 -131.21) (width 0.2) (layer "F.Cu") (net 3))
 (segment (start 35.88 -127.955) (end 35.88 -124.785) (width 0.2) (layer "F.Cu") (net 3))
 (segment (start 43.18 -130.81) (end 43.796 -130.81) (width 0.2) (layer "F.Cu") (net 3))
 (segment (start 39.37 -129.159) (end 38.481 -128.27) (width 0.2) (layer "F.Cu") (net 3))
 (via (at 43.18 -130.81) (size 0.6) (drill 0.3) (layers "F.Cu" "B.Cu") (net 3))
 (via (at 40.005 -129.159) (size 0.6) (drill 0.3) (layers "F.Cu" "B.Cu") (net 3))
 (segment (start 43.18 -130.175) (end 43.18 -130.81) (width 0.2) (layer "B.Cu") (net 3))
 (segment (start 40.005 -129.159) (end 42.164 -129.159) (width 0.2) (layer "B.Cu") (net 3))
 (segment (start 42.164 -129.159) (end 43.18 -130.175) (width 0.2) (layer "B.Cu") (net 3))
 (segment (start 31.88 -128.527) (end 32.37 -129.017) (width 0.2) (layer "F.Cu") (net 1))
 (segment (start 32.37 -129.017) (end 32.37 -129.987) (width 0.2) (layer "F.Cu") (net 1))
 (segment (start 31.88 -124.785) (end 31.88 -128.527) (width 0.2) (layer "F.Cu") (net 1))
 (segment (start 33.6295 -136.271) (end 32.067 -136.271) (width 0.2) (layer "F.Cu") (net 21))
 (segment (start 32.067 -136.271) (end 32.004 -136.334) (width 0.2) (layer "F.Cu") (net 21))
 (segment (start 33.88 -129.315) (end 33.88 -124.785) (width 0.2) (layer "F.Cu") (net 2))
 (segment (start 33.67 -129.987) (end 33.67 -129.525) (width 0.2) (layer "F.Cu") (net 2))
 (segment (start 33.67 -129.525) (end 33.88 -129.315) (width 0.2) (layer "F.Cu") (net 2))
 (segment (start 44.2965 -135.889) (end 44.196 -135.7885) (width 0.2) (layer "F.Cu") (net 22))
 (segment (start 45.72 -135.889) (end 44.2965 -135.889) (width 0.2) (layer "F.Cu") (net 22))
 (segment (start 41.006 -129.779) (end 40.64 -129.413) (width 0.2) (layer "F.Cu") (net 8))
 (segment (start 45.72 -128.143) (end 45.847 -128.016) (width 0.2) (layer "F.Cu") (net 8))
 (segment (start 40.64 -129.413) (end 40.64 -128.651) (width 0.2) (layer "F.Cu") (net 8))
 (segment (start 45.88 -127.983) (end 45.88 -124.785) (width 0.2) (layer "F.Cu") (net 8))
 (segment (start 45.847 -128.016) (end 45.88 -127.983) (width 0.2) (layer "F.Cu") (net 8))
 (segment (start 40.64 -128.651) (end 41.148 -128.143) (width 0.2) (layer "F.Cu") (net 8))
 (segment (start 41.148 -128.143) (end 45.72 -128.143) (width 0.2) (layer "F.Cu") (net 8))
 (segment (start 41.006 -129.987) (end 41.006 -129.779) (width 0.2) (layer "F.Cu") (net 8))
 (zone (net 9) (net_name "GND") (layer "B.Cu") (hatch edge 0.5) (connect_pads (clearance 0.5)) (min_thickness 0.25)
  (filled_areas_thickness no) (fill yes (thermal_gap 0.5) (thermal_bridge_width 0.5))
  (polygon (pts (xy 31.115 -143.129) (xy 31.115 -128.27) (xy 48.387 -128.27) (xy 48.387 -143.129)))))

